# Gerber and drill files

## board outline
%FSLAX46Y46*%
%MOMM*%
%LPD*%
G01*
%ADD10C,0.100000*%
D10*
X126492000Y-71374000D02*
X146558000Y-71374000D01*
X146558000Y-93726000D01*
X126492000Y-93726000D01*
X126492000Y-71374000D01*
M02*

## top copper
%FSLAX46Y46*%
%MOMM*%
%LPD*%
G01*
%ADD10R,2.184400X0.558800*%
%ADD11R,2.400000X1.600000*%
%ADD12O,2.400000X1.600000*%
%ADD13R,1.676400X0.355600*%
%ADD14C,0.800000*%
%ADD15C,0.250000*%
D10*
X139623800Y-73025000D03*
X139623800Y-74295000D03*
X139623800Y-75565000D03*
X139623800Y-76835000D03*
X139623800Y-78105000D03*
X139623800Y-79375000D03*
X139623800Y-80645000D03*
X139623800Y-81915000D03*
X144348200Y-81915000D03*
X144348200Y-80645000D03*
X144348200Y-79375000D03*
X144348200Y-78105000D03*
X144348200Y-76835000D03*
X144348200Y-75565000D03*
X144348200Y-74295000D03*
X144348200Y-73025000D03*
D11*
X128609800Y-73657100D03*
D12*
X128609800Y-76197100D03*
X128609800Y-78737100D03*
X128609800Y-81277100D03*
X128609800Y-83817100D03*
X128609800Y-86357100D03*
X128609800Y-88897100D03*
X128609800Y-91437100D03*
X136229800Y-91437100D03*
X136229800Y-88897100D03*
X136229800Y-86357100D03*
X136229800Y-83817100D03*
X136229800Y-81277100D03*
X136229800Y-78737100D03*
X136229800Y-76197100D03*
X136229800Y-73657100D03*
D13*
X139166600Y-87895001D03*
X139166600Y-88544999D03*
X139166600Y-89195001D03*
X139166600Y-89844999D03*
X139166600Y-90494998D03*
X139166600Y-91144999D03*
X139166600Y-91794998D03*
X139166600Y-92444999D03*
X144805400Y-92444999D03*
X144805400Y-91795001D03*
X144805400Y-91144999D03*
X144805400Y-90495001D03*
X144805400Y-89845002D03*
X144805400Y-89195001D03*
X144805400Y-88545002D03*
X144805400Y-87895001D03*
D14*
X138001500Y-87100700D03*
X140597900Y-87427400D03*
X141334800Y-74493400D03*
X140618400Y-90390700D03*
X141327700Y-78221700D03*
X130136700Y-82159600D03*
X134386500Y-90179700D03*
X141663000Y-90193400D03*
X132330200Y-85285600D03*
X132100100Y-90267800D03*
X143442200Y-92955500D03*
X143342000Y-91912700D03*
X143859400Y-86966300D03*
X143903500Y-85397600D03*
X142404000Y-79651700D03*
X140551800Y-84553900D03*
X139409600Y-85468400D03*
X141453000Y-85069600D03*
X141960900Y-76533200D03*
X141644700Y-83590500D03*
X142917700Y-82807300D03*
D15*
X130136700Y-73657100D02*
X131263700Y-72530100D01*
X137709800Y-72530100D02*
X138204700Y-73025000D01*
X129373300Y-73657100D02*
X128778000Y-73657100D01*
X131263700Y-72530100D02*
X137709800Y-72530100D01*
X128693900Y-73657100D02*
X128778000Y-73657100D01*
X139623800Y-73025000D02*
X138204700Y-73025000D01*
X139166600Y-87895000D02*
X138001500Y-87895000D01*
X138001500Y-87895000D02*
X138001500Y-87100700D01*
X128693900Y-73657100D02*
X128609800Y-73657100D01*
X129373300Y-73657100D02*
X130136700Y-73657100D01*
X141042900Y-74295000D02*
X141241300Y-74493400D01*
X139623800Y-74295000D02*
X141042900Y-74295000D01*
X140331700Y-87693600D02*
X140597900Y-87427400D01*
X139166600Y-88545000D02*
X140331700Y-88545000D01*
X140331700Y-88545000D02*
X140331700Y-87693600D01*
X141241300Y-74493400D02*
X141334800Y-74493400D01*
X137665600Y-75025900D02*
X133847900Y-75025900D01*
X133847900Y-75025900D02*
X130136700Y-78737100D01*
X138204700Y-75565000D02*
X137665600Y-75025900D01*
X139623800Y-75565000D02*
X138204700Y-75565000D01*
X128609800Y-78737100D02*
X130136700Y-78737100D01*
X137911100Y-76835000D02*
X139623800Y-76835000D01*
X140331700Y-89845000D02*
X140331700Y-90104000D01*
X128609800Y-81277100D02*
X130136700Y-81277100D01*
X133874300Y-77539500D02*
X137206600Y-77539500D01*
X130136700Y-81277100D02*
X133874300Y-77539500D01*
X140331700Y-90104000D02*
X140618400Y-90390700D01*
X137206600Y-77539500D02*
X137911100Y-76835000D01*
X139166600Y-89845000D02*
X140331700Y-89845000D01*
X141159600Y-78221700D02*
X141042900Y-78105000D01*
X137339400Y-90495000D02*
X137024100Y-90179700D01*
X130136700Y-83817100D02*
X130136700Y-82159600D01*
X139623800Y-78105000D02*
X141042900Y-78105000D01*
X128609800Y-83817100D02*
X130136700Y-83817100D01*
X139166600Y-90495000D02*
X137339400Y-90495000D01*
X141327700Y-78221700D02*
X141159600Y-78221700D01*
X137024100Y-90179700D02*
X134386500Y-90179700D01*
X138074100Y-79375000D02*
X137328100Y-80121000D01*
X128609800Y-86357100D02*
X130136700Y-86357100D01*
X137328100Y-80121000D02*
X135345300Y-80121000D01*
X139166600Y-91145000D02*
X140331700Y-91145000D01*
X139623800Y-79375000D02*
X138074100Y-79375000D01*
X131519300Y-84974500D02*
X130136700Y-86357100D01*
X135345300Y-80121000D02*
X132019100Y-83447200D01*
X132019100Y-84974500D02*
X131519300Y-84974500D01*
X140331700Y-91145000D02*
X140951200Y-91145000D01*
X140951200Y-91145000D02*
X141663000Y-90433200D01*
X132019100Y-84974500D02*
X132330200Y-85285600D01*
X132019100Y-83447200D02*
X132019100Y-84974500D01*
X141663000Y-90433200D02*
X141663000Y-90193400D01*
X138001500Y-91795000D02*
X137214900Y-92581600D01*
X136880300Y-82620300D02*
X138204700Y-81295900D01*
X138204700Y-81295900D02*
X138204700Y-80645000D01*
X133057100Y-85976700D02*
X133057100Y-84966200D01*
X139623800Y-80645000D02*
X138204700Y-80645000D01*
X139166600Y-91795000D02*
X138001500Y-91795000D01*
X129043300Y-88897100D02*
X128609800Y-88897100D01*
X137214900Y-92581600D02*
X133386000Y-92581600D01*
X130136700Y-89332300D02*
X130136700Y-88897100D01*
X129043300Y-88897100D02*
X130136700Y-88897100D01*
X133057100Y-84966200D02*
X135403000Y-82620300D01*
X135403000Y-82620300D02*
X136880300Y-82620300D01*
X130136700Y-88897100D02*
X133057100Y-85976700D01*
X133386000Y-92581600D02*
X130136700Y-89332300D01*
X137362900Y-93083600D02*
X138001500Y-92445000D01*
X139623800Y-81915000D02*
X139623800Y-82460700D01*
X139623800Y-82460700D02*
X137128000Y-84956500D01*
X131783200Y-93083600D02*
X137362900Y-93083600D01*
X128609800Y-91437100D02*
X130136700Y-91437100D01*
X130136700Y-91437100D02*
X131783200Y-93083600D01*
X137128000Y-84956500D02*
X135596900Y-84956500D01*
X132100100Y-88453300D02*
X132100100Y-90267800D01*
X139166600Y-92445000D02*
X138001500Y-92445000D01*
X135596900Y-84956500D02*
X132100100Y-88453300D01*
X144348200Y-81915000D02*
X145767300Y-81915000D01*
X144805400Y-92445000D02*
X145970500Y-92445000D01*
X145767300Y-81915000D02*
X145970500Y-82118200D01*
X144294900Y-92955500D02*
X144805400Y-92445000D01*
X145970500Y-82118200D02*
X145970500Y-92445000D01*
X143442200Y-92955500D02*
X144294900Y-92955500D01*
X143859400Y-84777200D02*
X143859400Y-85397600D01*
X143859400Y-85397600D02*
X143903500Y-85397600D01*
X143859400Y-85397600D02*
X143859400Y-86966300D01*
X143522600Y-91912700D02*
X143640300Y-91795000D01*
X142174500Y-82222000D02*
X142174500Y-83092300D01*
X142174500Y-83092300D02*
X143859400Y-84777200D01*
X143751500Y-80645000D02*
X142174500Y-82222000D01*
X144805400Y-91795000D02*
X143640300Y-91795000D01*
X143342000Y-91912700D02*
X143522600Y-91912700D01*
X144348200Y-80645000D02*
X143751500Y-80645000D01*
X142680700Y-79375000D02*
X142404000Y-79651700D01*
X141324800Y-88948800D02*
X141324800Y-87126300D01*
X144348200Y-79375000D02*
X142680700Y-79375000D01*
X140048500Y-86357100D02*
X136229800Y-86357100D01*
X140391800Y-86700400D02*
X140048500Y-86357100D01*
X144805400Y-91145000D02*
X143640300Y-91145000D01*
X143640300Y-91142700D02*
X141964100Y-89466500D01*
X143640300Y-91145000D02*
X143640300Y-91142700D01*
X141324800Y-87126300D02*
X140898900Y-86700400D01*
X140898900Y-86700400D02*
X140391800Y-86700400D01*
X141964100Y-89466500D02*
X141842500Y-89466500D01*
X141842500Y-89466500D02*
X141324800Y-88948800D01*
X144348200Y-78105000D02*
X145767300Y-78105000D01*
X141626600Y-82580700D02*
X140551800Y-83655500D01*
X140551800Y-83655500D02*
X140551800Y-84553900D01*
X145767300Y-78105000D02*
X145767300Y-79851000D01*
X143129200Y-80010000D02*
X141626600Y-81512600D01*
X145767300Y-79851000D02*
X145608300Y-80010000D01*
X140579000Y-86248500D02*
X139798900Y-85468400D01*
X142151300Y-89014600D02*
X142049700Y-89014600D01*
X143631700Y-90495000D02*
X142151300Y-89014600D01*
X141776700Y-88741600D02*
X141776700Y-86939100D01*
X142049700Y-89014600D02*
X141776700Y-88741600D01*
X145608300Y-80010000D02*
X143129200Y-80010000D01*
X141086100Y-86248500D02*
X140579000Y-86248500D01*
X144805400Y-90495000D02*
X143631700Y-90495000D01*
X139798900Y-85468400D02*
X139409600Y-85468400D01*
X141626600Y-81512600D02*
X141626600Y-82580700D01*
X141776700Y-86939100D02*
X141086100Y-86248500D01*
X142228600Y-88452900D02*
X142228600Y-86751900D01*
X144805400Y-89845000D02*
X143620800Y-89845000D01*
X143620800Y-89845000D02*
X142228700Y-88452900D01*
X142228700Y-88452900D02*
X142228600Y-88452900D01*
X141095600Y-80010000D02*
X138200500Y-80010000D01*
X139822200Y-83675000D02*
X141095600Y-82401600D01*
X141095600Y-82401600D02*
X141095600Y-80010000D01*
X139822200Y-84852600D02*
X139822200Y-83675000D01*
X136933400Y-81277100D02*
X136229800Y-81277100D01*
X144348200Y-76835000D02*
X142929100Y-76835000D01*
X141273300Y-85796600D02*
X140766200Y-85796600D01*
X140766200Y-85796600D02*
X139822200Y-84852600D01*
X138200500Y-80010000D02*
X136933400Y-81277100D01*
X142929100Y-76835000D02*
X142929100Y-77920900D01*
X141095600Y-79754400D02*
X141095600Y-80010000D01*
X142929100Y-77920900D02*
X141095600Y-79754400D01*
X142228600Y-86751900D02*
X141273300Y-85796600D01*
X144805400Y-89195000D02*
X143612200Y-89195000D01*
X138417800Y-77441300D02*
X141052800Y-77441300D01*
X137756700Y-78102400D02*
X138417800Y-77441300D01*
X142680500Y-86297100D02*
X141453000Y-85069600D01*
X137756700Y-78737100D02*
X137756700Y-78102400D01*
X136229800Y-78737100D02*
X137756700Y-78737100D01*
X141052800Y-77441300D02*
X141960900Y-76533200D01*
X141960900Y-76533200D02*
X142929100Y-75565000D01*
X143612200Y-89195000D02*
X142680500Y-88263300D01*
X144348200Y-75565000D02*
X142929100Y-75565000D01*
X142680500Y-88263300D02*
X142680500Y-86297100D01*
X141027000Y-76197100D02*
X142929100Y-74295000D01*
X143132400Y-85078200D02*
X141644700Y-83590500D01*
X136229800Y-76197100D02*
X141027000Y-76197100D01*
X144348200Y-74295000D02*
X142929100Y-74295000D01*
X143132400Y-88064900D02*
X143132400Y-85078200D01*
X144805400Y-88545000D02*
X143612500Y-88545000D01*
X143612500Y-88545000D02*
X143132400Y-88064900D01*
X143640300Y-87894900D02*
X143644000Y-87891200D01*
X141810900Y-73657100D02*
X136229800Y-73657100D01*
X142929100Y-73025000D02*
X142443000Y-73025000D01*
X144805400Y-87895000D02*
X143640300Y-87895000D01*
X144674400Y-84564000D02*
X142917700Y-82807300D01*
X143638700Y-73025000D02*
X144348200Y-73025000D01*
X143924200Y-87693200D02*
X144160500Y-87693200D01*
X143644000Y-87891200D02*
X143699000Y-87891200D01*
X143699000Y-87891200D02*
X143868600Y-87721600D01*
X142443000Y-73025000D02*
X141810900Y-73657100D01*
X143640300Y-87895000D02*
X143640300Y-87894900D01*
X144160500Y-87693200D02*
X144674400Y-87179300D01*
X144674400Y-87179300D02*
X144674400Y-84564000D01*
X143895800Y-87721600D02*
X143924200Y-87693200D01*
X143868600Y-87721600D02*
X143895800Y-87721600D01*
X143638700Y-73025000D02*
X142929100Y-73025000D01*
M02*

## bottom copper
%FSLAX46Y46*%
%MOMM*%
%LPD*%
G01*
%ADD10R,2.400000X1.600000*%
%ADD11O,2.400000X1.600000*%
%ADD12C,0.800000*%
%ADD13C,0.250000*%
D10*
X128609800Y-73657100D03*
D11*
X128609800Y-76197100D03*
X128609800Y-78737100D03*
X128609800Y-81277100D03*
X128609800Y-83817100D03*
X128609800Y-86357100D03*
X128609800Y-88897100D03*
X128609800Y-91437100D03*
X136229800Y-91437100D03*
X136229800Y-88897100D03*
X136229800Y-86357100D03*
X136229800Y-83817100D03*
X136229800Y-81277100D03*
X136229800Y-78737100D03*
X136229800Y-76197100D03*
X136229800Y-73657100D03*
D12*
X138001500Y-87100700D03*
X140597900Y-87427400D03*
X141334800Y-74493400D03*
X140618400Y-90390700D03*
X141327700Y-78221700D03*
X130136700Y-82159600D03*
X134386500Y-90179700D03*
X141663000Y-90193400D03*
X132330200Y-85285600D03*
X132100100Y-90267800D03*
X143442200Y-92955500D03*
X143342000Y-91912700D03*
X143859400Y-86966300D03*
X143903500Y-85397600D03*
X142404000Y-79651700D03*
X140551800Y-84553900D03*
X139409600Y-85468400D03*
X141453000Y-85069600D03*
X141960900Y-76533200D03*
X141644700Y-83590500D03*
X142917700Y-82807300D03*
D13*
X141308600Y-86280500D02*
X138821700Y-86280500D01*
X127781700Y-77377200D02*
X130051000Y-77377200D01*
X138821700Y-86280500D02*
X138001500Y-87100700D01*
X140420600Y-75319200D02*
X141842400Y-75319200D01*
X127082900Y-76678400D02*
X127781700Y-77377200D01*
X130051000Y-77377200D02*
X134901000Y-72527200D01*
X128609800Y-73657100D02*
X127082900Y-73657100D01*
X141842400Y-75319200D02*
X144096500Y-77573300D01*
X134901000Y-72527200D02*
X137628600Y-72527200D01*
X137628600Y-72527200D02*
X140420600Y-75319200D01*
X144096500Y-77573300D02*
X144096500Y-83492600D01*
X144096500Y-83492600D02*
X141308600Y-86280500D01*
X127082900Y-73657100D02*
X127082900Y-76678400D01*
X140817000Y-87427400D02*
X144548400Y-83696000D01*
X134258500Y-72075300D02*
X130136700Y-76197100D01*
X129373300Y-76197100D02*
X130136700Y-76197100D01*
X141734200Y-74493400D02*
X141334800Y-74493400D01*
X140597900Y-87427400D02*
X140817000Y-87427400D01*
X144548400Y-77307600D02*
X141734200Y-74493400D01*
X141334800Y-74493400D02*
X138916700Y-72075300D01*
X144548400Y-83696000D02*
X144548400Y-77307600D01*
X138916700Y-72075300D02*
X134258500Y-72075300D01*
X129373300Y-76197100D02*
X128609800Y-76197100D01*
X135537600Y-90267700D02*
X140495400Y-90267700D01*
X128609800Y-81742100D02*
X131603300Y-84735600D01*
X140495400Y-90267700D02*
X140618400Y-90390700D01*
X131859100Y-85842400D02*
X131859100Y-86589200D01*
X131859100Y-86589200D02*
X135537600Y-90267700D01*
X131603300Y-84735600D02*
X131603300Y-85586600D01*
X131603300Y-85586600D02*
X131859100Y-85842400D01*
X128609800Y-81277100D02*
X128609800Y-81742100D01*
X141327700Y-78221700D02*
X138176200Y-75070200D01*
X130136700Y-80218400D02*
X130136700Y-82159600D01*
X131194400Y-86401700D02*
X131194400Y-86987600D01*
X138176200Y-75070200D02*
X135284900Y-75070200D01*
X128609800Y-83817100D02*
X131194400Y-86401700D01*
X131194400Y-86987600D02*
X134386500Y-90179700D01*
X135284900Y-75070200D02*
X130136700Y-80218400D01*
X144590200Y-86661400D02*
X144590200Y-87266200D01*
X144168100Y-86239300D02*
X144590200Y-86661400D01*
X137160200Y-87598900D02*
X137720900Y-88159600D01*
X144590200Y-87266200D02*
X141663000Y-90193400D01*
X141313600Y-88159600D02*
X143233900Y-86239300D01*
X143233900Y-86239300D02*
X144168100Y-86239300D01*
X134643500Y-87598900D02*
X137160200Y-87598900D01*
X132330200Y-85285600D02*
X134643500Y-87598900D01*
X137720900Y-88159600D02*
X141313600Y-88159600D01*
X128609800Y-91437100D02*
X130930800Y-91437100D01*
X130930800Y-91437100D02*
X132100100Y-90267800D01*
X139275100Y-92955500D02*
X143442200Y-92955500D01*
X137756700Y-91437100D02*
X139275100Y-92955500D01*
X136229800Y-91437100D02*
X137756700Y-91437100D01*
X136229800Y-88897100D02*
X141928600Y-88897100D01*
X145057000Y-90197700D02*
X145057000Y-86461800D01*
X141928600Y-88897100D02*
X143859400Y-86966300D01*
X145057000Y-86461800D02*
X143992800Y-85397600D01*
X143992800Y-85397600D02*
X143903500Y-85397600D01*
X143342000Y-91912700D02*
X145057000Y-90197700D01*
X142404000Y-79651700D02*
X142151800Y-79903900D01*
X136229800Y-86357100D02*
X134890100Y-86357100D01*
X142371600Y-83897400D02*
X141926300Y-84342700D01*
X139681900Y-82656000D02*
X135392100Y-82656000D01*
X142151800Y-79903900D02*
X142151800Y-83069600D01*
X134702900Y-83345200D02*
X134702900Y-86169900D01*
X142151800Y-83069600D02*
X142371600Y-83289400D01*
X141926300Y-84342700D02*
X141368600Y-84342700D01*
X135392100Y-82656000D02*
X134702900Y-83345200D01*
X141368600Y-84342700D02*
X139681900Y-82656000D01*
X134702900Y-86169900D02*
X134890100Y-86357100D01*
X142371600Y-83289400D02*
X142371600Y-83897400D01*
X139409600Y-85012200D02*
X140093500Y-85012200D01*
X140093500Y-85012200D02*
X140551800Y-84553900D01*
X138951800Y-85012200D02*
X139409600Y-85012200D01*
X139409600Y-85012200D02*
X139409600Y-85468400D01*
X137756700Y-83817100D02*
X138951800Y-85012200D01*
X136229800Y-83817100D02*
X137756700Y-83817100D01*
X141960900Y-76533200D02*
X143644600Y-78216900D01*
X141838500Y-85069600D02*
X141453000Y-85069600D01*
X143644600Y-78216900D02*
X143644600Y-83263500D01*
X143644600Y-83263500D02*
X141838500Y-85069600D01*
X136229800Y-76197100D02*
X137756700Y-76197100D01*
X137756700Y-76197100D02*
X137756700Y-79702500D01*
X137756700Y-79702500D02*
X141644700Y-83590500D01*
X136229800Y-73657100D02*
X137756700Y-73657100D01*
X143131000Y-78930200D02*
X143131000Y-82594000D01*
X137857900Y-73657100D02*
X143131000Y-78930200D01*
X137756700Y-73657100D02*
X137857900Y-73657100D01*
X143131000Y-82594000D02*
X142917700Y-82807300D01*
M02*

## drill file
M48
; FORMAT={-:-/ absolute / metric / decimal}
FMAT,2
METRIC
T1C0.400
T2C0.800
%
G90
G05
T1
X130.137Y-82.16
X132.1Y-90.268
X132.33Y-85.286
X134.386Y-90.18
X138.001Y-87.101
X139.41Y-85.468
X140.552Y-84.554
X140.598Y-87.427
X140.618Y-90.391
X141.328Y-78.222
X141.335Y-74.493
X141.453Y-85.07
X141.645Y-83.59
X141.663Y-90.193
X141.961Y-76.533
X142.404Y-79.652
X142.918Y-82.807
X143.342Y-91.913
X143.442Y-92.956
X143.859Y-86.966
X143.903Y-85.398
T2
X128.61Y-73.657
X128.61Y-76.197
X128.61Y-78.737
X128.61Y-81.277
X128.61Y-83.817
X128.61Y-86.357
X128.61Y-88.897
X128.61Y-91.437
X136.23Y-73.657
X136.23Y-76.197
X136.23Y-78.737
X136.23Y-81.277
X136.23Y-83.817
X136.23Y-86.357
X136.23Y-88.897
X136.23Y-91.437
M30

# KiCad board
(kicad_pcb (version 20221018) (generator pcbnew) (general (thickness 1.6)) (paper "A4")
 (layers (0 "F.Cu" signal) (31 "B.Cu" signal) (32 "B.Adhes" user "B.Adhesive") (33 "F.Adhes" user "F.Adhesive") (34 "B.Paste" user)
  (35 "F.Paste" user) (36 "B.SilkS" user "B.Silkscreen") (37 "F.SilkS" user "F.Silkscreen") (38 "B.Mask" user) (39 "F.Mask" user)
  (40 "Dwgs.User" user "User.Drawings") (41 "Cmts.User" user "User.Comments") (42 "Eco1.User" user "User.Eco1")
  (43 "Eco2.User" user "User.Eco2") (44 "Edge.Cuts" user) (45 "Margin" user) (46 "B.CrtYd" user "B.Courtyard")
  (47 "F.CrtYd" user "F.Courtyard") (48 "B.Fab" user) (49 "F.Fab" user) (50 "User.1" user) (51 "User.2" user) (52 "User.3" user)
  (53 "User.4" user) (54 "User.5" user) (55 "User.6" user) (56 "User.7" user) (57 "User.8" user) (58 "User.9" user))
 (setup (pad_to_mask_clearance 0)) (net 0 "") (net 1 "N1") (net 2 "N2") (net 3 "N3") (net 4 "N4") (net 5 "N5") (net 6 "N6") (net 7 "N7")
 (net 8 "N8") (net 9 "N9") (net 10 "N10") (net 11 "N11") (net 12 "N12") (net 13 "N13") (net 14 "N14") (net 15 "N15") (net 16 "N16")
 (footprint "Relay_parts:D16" (layer "F.Cu") (at 141.986 77.47)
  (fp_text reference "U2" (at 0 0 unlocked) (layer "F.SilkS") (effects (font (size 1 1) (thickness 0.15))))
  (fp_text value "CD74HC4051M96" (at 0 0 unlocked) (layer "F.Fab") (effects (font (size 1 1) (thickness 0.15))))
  (pad "1" smd rect (at -2.3622 -4.445) (size 2.1844 0.5588) (layers "F.Cu" "F.Paste" "F.Mask") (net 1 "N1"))
  (pad "2" smd rect (at -2.3622 -3.175) (size 2.1844 0.5588) (layers "F.Cu" "F.Paste" "F.Mask") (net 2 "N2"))
  (pad "3" smd rect (at -2.3622 -1.905) (size 2.1844 0.5588) (layers "F.Cu" "F.Paste" "F.Mask") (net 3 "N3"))
  (pad "4" smd rect (at -2.3622 -0.635) (size 2.1844 0.5588) (layers "F.Cu" "F.Paste" "F.Mask") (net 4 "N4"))
  (pad "5" smd rect (at -2.3622 0.635) (size 2.1844 0.5588) (layers "F.Cu" "F.Paste" "F.Mask") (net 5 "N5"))
  (pad "6" smd rect (at -2.3622 1.905) (size 2.1844 0.5588) (layers "F.Cu" "F.Paste" "F.Mask") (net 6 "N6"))
  (pad "7" smd rect (at -2.3622 3.175) (size 2.1844 0.5588) (layers "F.Cu" "F.Paste" "F.Mask") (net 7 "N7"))
  (pad "8" smd rect (at -2.3622 4.445) (size 2.1844 0.5588) (layers "F.Cu" "F.Paste" "F.Mask") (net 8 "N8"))
  (pad "9" smd rect (at 2.3622 4.445) (size 2.1844 0.5588) (layers "F.Cu" "F.Paste" "F.Mask") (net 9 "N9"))
  (pad "10" smd rect (at 2.3622 3.175) (size 2.1844 0.5588) (layers "F.Cu" "F.Paste" "F.Mask") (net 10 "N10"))
  (pad "11" smd rect (at 2.3622 1.905) (size 2.1844 0.5588) (layers "F.Cu" "F.Paste" "F.Mask") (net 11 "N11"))
  (pad "12" smd rect (at 2.3622 0.635) (size 2.1844 0.5588) (layers "F.Cu" "F.Paste" "F.Mask") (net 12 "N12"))
  (pad "13" smd rect (at 2.3622 -0.635) (size 2.1844 0.5588) (layers "F.Cu" "F.Paste" "F.Mask") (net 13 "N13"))
  (pad "14" smd rect (at 2.3622 -1.905) (size 2.1844 0.5588) (layers "F.Cu" "F.Paste" "F.Mask") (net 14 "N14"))
  (pad "15" smd rect (at 2.3622 -3.175) (size 2.1844 0.5588) (layers "F.Cu" "F.Paste" "F.Mask") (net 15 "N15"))
  (pad "16" smd rect (at 2.3622 -4.445) (size 2.1844 0.5588) (layers "F.Cu" "F.Paste" "F.Mask") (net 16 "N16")))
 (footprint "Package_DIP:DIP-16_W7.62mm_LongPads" (layer "F.Cu") (at 128.6098 73.6571)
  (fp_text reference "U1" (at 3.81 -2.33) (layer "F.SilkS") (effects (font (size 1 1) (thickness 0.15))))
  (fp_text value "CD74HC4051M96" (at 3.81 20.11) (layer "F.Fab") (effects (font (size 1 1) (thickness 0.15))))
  (pad "1" thru_hole rect (at 0 0) (size 2.4 1.6) (drill 0.8) (layers "*.Cu" "*.Mask") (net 1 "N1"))
  (pad "2" thru_hole oval (at 0 2.54) (size 2.4 1.6) (drill 0.8) (layers "*.Cu" "*.Mask") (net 2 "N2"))
  (pad "3" thru_hole oval (at 0 5.08) (size 2.4 1.6) (drill 0.8) (layers "*.Cu" "*.Mask") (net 3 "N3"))
  (pad "4" thru_hole oval (at 0 7.62) (size 2.4 1.6) (drill 0.8) (layers "*.Cu" "*.Mask") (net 4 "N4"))
  (pad "5" thru_hole oval (at 0 10.16) (size 2.4 1.6) (drill 0.8) (layers "*.Cu" "*.Mask") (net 5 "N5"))
  (pad "6" thru_hole oval (at 0 12.7) (size 2.4 1.6) (drill 0.8) (layers "*.Cu" "*.Mask") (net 6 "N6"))
  (pad "7" thru_hole oval (at 0 15.24) (size 2.4 1.6) (drill 0.8) (layers "*.Cu" "*.Mask") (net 7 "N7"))
  (pad "8" thru_hole oval (at 0 17.78) (size 2.4 1.6) (drill 0.8) (layers "*.Cu" "*.Mask") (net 8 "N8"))
  (pad "9" thru_hole oval (at 7.62 17.78) (size 2.4 1.6) (drill 0.8) (layers "*.Cu" "*.Mask") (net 9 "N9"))
  (pad "10" thru_hole oval (at 7.62 15.24) (size 2.4 1.6) (drill 0.8) (layers "*.Cu" "*.Mask") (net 10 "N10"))
  (pad "11" thru_hole oval (at 7.62 12.7) (size 2.4 1.6) (drill 0.8) (layers "*.Cu" "*.Mask") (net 11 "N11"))
  (pad "12" thru_hole oval (at 7.62 10.16) (size 2.4 1.6) (drill 0.8) (layers "*.Cu" "*.Mask") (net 12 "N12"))
  (pad "13" thru_hole oval (at 7.62 7.62) (size 2.4 1.6) (drill 0.8) (layers "*.Cu" "*.Mask") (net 13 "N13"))
  (pad "14" thru_hole oval (at 7.62 5.08) (size 2.4 1.6) (drill 0.8) (layers "*.Cu" "*.Mask") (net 14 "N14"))
  (pad "15" thru_hole oval (at 7.62 2.54) (size 2.4 1.6) (drill 0.8) (layers "*.Cu" "*.Mask") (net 15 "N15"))
  (pad "16" thru_hole oval (at 7.62 0) (size 2.4 1.6) (drill 0.8) (layers "*.Cu" "*.Mask") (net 16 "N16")))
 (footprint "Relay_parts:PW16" (layer "F.Cu") (at 141.986 90.17)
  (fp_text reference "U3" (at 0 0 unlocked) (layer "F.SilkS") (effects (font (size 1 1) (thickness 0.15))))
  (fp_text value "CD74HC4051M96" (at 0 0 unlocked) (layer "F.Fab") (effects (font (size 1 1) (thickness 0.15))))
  (pad "1" smd rect (at -2.8194 -2.274999) (size 1.6764 0.3556) (layers "F.Cu" "F.Paste" "F.Mask") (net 1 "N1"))
  (pad "2" smd rect (at -2.8194 -1.625001) (size 1.6764 0.3556) (layers "F.Cu" "F.Paste" "F.Mask") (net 2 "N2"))
  (pad "3" smd rect (at -2.8194 -0.974999) (size 1.6764 0.3556) (layers "F.Cu" "F.Paste" "F.Mask") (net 3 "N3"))
  (pad "4" smd rect (at -2.8194 -0.325001) (size 1.6764 0.3556) (layers "F.Cu" "F.Paste" "F.Mask") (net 4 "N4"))
  (pad "5" smd rect (at -2.8194 0.324998) (size 1.6764 0.3556) (layers "F.Cu" "F.Paste" "F.Mask") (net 5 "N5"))
  (pad "6" smd rect (at -2.8194 0.974999) (size 1.6764 0.3556) (layers "F.Cu" "F.Paste" "F.Mask") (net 6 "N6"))
  (pad "7" smd rect (at -2.8194 1.624998) (size 1.6764 0.3556) (layers "F.Cu" "F.Paste" "F.Mask") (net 7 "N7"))
  (pad "8" smd rect (at -2.8194 2.274999) (size 1.6764 0.3556) (layers "F.Cu" "F.Paste" "F.Mask") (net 8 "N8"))
  (pad "9" smd rect (at 2.8194 2.274999) (size 1.6764 0.3556) (layers "F.Cu" "F.Paste" "F.Mask") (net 9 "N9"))
  (pad "10" smd rect (at 2.8194 1.625001) (size 1.6764 0.3556) (layers "F.Cu" "F.Paste" "F.Mask") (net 10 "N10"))
  (pad "11" smd rect (at 2.8194 0.974999) (size 1.6764 0.3556) (layers "F.Cu" "F.Paste" "F.Mask") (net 11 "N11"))
  (pad "12" smd rect (at 2.8194 0.325001) (size 1.6764 0.3556) (layers "F.Cu" "F.Paste" "F.Mask") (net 12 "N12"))
  (pad "13" smd rect (at 2.8194 -0.324998) (size 1.6764 0.3556) (layers "F.Cu" "F.Paste" "F.Mask") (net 13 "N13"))
  (pad "14" smd rect (at 2.8194 -0.974999) (size 1.6764 0.3556) (layers "F.Cu" "F.Paste" "F.Mask") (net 14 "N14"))
  (pad "15" smd rect (at 2.8194 -1.624998) (size 1.6764 0.3556) (layers "F.Cu" "F.Paste" "F.Mask") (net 15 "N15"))
  (pad "16" smd rect (at 2.8194 -2.274999) (size 1.6764 0.3556) (layers "F.Cu" "F.Paste" "F.Mask") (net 16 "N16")))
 (gr_rect (start 126.492 71.374) (end 146.558 93.726) (stroke (width 0.1) (type default)) (fill none) (layer "Edge.Cuts"))
 (segment (start 130.1367 73.6571) (end 131.2637 72.5301) (width 0.25) (layer "F.Cu") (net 1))
 (segment (start 137.7098 72.5301) (end 138.2047 73.025) (width 0.25) (layer "F.Cu") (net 1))
 (segment (start 129.3733 73.6571) (end 128.778 73.6571) (width 0.25) (layer "F.Cu") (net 1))
 (segment (start 131.2637 72.5301) (end 137.7098 72.5301) (width 0.25) (layer "F.Cu") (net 1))
 (segment (start 128.6939 73.6571) (end 128.778 73.6571) (width 0.25) (layer "F.Cu") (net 1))
 (segment (start 139.6238 73.025) (end 138.2047 73.025) (width 0.25) (layer "F.Cu") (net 1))
 (segment (start 139.1666 87.895) (end 138.0015 87.895) (width 0.25) (layer "F.Cu") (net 1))
 (segment (start 138.0015 87.895) (end 138.0015 87.1007) (width 0.25) (layer "F.Cu") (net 1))
 (segment (start 128.6939 73.6571) (end 128.6098 73.6571) (width 0.25) (layer "F.Cu") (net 1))
 (segment (start 129.3733 73.6571) (end 130.1367 73.6571) (width 0.25) (layer "F.Cu") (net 1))
 (via (at 138.0015 87.1007) (size 0.8) (drill 0.4) (layers "F.Cu" "B.Cu") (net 1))
 (segment (start 141.3086 86.2805) (end 138.8217 86.2805) (width 0.25) (layer "B.Cu") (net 1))
 (segment (start 127.7817 77.3772) (end 130.051 77.3772) (width 0.25) (layer "B.Cu") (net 1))
 (segment (start 138.8217 86.2805) (end 138.0015 87.1007) (width 0.25) (layer "B.Cu") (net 1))
 (segment (start 140.4206 75.3192) (end 141.8424 75.3192) (width 0.25) (layer "B.Cu") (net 1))
 (segment (start 127.0829 76.6784) (end 127.7817 77.3772) (width 0.25) (layer "B.Cu") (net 1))
 (segment (start 130.051 77.3772) (end 134.901 72.5272) (width 0.25) (layer "B.Cu") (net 1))
 (segment (start 128.6098 73.6571) (end 127.0829 73.6571) (width 0.25) (layer "B.Cu") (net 1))
 (segment (start 141.8424 75.3192) (end 144.0965 77.5733) (width 0.25) (layer "B.Cu") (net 1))
 (segment (start 134.901 72.5272) (end 137.6286 72.5272) (width 0.25) (layer "B.Cu") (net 1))
 (segment (start 137.6286 72.5272) (end 140.4206 75.3192) (width 0.25) (layer "B.Cu") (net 1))
 (segment (start 144.0965 77.5733) (end 144.0965 83.4926) (width 0.25) (layer "B.Cu") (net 1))
 (segment (start 144.0965 83.4926) (end 141.3086 86.2805) (width 0.25) (layer "B.Cu") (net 1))
 (segment (start 127.0829 73.6571) (end 127.0829 76.6784) (width 0.25) (layer "B.Cu") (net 1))
 (segment (start 141.0429 74.295) (end 141.2413 74.4934) (width 0.25) (layer "F.Cu") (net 2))
 (segment (start 139.6238 74.295) (end 141.0429 74.295) (width 0.25) (layer "F.Cu") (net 2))
 (segment (start 140.3317 87.6936) (end 140.5979 87.4274) (width 0.25) (layer "F.Cu") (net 2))
 (segment (start 139.1666 88.545) (end 140.3317 88.545) (width 0.25) (layer "F.Cu") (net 2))
 (segment (start 140.3317 88.545) (end 140.3317 87.6936) (width 0.25) (layer "F.Cu") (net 2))
 (segment (start 141.2413 74.4934) (end 141.3348 74.4934) (width 0.25) (layer "F.Cu") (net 2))
 (via (at 140.5979 87.4274) (size 0.8) (drill 0.4) (layers "F.Cu" "B.Cu") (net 2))
 (via (at 141.3348 74.4934) (size 0.8) (drill 0.4) (layers "F.Cu" "B.Cu") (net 2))
 (segment (start 140.817 87.4274) (end 144.5484 83.696) (width 0.25) (layer "B.Cu") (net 2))
 (segment (start 134.2585 72.0753) (end 130.1367 76.1971) (width 0.25) (layer "B.Cu") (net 2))
 (segment (start 129.3733 76.1971) (end 130.1367 76.1971) (width 0.25) (layer "B.Cu") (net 2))
 (segment (start 141.7342 74.4934) (end 141.3348 74.4934) (width 0.25) (layer "B.Cu") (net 2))
 (segment (start 140.5979 87.4274) (end 140.817 87.4274) (width 0.25) (layer "B.Cu") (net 2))
 (segment (start 144.5484 77.3076) (end 141.7342 74.4934) (width 0.25) (layer "B.Cu") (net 2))
 (segment (start 141.3348 74.4934) (end 138.9167 72.0753) (width 0.25) (layer "B.Cu") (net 2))
 (segment (start 144.5484 83.696) (end 144.5484 77.3076) (width 0.25) (layer "B.Cu") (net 2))
 (segment (start 138.9167 72.0753) (end 134.2585 72.0753) (width 0.25) (layer "B.Cu") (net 2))
 (segment (start 129.3733 76.1971) (end 128.6098 76.1971) (width 0.25) (layer "B.Cu") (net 2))
 (segment (start 137.6656 75.0259) (end 133.8479 75.0259) (width 0.25) (layer "F.Cu") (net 3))
 (segment (start 133.8479 75.0259) (end 130.1367 78.7371) (width 0.25) (layer "F.Cu") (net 3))
 (segment (start 138.2047 75.565) (end 137.6656 75.0259) (width 0.25) (layer "F.Cu") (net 3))
 (segment (start 139.6238 75.565) (end 138.2047 75.565) (width 0.25) (layer "F.Cu") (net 3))
 (segment (start 128.6098 78.7371) (end 130.1367 78.7371) (width 0.25) (layer "F.Cu") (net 3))
 (segment (start 137.9111 76.835) (end 139.6238 76.835) (width 0.25) (layer "F.Cu") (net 4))
 (segment (start 140.3317 89.845) (end 140.3317 90.104) (width 0.25) (layer "F.Cu") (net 4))
 (segment (start 128.6098 81.2771) (end 130.1367 81.2771) (width 0.25) (layer "F.Cu") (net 4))
 (segment (start 133.8743 77.5395) (end 137.2066 77.5395) (width 0.25) (layer "F.Cu") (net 4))
 (segment (start 130.1367 81.2771) (end 133.8743 77.5395) (width 0.25) (layer "F.Cu") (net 4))
 (segment (start 140.3317 90.104) (end 140.6184 90.3907) (width 0.25) (layer "F.Cu") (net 4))
 (segment (start 137.2066 77.5395) (end 137.9111 76.835) (width 0.25) (layer "F.Cu") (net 4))
 (segment (start 139.1666 89.845) (end 140.3317 89.845) (width 0.25) (layer "F.Cu") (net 4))
 (via (at 140.6184 90.3907) (size 0.8) (drill 0.4) (layers "F.Cu" "B.Cu") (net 4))
 (segment (start 135.5376 90.2677) (end 140.4954 90.2677) (width 0.25) (layer "B.Cu") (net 4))
 (segment (start 128.6098 81.7421) (end 131.6033 84.7356) (width 0.25) (layer "B.Cu") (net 4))
 (segment (start 140.4954 90.2677) (end 140.6184 90.3907) (width 0.25) (layer "B.Cu") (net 4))
 (segment (start 131.8591 85.8424) (end 131.8591 86.5892) (width 0.25) (layer "B.Cu") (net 4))
 (segment (start 131.8591 86.5892) (end 135.5376 90.2677) (width 0.25) (layer "B.Cu") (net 4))
 (segment (start 131.6033 84.7356) (end 131.6033 85.5866) (width 0.25) (layer "B.Cu") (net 4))
 (segment (start 131.6033 85.5866) (end 131.8591 85.8424) (width 0.25) (layer "B.Cu") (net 4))
 (segment (start 128.6098 81.2771) (end 128.6098 81.7421) (width 0.25) (layer "B.Cu") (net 4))
 (segment (start 141.1596 78.2217) (end 141.0429 78.105) (width 0.25) (layer "F.Cu") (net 5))
 (segment (start 137.3394 90.495) (end 137.0241 90.1797) (width 0.25) (layer "F.Cu") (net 5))
 (segment (start 130.1367 83.8171) (end 130.1367 82.1596) (width 0.25) (layer "F.Cu") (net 5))
 (segment (start 139.6238 78.105) (end 141.0429 78.105) (width 0.25) (layer "F.Cu") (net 5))
 (segment (start 128.6098 83.8171) (end 130.1367 83.8171) (width 0.25) (layer "F.Cu") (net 5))
 (segment (start 139.1666 90.495) (end 137.3394 90.495) (width 0.25) (layer "F.Cu") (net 5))
 (segment (start 141.3277 78.2217) (end 141.1596 78.2217) (width 0.25) (layer "F.Cu") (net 5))
 (segment (start 137.0241 90.1797) (end 134.3865 90.1797) (width 0.25) (layer "F.Cu") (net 5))
 (via (at 141.3277 78.2217) (size 0.8) (drill 0.4) (layers "F.Cu" "B.Cu") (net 5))
 (via (at 130.1367 82.1596) (size 0.8) (drill 0.4) (layers "F.Cu" "B.Cu") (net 5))
 (via (at 134.3865 90.1797) (size 0.8) (drill 0.4) (layers "F.Cu" "B.Cu") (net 5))
 (segment (start 141.3277 78.2217) (end 138.1762 75.0702) (width 0.25) (layer "B.Cu") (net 5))
 (segment (start 130.1367 80.2184) (end 130.1367 82.1596) (width 0.25) (layer "B.Cu") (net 5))
 (segment (start 131.1944 86.4017) (end 131.1944 86.9876) (width 0.25) (layer "B.Cu") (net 5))
 (segment (start 138.1762 75.0702) (end 135.2849 75.0702) (width 0.25) (layer "B.Cu") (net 5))
 (segment (start 128.6098 83.8171) (end 131.1944 86.4017) (width 0.25) (layer "B.Cu") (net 5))
 (segment (start 131.1944 86.9876) (end 134.3865 90.1797) (width 0.25) (layer "B.Cu") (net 5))
 (segment (start 135.2849 75.0702) (end 130.1367 80.2184) (width 0.25) (layer "B.Cu") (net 5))
 (segment (start 138.0741 79.375) (end 137.3281 80.121) (width 0.25) (layer "F.Cu") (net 6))
 (segment (start 128.6098 86.3571) (end 130.1367 86.3571) (width 0.25) (layer "F.Cu") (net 6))
 (segment (start 137.3281 80.121) (end 135.3453 80.121) (width 0.25) (layer "F.Cu") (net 6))
 (segment (start 139.1666 91.145) (end 140.3317 91.145) (width 0.25) (layer "F.Cu") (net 6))
 (segment (start 139.6238 79.375) (end 138.0741 79.375) (width 0.25) (layer "F.Cu") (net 6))
 (segment (start 131.5193 84.9745) (end 130.1367 86.3571) (width 0.25) (layer "F.Cu") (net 6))
 (segment (start 135.3453 80.121) (end 132.0191 83.4472) (width 0.25) (layer "F.Cu") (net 6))
 (segment (start 132.0191 84.9745) (end 131.5193 84.9745) (width 0.25) (layer "F.Cu") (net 6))
 (segment (start 140.3317 91.145) (end 140.9512 91.145) (width 0.25) (layer "F.Cu") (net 6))
 (segment (start 140.9512 91.145) (end 141.663 90.4332) (width 0.25) (layer "F.Cu") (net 6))
 (segment (start 132.0191 84.9745) (end 132.3302 85.2856) (width 0.25) (layer "F.Cu") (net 6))
 (segment (start 132.0191 83.4472) (end 132.0191 84.9745) (width 0.25) (layer "F.Cu") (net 6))
 (segment (start 141.663 90.4332) (end 141.663 90.1934) (width 0.25) (layer "F.Cu") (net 6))
 (via (at 141.663 90.1934) (size 0.8) (drill 0.4) (layers "F.Cu" "B.Cu") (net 6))
 (via (at 132.3302 85.2856) (size 0.8) (drill 0.4) (layers "F.Cu" "B.Cu") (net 6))
 (segment (start 144.5902 86.6614) (end 144.5902 87.2662) (width 0.25) (layer "B.Cu") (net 6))
 (segment (start 144.1681 86.2393) (end 144.5902 86.6614) (width 0.25) (layer "B.Cu") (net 6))
 (segment (start 137.1602 87.5989) (end 137.7209 88.1596) (width 0.25) (layer "B.Cu") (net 6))
 (segment (start 144.5902 87.2662) (end 141.663 90.1934) (width 0.25) (layer "B.Cu") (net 6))
 (segment (start 141.3136 88.1596) (end 143.2339 86.2393) (width 0.25) (layer "B.Cu") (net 6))
 (segment (start 143.2339 86.2393) (end 144.1681 86.2393) (width 0.25) (layer "B.Cu") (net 6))
 (segment (start 134.6435 87.5989) (end 137.1602 87.5989) (width 0.25) (layer "B.Cu") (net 6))
 (segment (start 132.3302 85.2856) (end 134.6435 87.5989) (width 0.25) (layer "B.Cu") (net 6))
 (segment (start 137.7209 88.1596) (end 141.3136 88.1596) (width 0.25) (layer "B.Cu") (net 6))
 (segment (start 138.0015 91.795) (end 137.2149 92.5816) (width 0.25) (layer "F.Cu") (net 7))
 (segment (start 136.8803 82.6203) (end 138.2047 81.2959) (width 0.25) (layer "F.Cu") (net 7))
 (segment (start 138.2047 81.2959) (end 138.2047 80.645) (width 0.25) (layer "F.Cu") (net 7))
 (segment (start 133.0571 85.9767) (end 133.0571 84.9662) (width 0.25) (layer "F.Cu") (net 7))
 (segment (start 139.6238 80.645) (end 138.2047 80.645) (width 0.25) (layer "F.Cu") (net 7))
 (segment (start 139.1666 91.795) (end 138.0015 91.795) (width 0.25) (layer "F.Cu") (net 7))
 (segment (start 129.0433 88.8971) (end 128.6098 88.8971) (width 0.25) (layer "F.Cu") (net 7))
 (segment (start 137.2149 92.5816) (end 133.386 92.5816) (width 0.25) (layer "F.Cu") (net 7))
 (segment (start 130.1367 89.3323) (end 130.1367 88.8971) (width 0.25) (layer "F.Cu") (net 7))
 (segment (start 129.0433 88.8971) (end 130.1367 88.8971) (width 0.25) (layer "F.Cu") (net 7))
 (segment (start 133.0571 84.9662) (end 135.403 82.6203) (width 0.25) (layer "F.Cu") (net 7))
 (segment (start 135.403 82.6203) (end 136.8803 82.6203) (width 0.25) (layer "F.Cu") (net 7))
 (segment (start 130.1367 88.8971) (end 133.0571 85.9767) (width 0.25) (layer "F.Cu") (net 7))
 (segment (start 133.386 92.5816) (end 130.1367 89.3323) (width 0.25) (layer "F.Cu") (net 7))
 (segment (start 137.3629 93.0836) (end 138.0015 92.445) (width 0.25) (layer "F.Cu") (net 8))
 (segment (start 139.6238 81.915) (end 139.6238 82.4607) (width 0.25) (layer "F.Cu") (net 8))
 (segment (start 139.6238 82.4607) (end 137.128 84.9565) (width 0.25) (layer "F.Cu") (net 8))
 (segment (start 131.7832 93.0836) (end 137.3629 93.0836) (width 0.25) (layer "F.Cu") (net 8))
 (segment (start 128.6098 91.4371) (end 130.1367 91.4371) (width 0.25) (layer "F.Cu") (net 8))
 (segment (start 130.1367 91.4371) (end 131.7832 93.0836) (width 0.25) (layer "F.Cu") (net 8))
 (segment (start 137.128 84.9565) (end 135.5969 84.9565) (width 0.25) (layer "F.Cu") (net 8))
 (segment (start 132.1001 88.4533) (end 132.1001 90.2678) (width 0.25) (layer "F.Cu") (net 8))
 (segment (start 139.1666 92.445) (end 138.0015 92.445) (width 0.25) (layer "F.Cu") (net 8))
 (segment (start 135.5969 84.9565) (end 132.1001 88.4533) (width 0.25) (layer "F.Cu") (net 8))
 (via (at 132.1001 90.2678) (size 0.8) (drill 0.4) (layers "F.Cu" "B.Cu") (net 8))
 (segment (start 128.6098 91.4371) (end 130.9308 91.4371) (width 0.25) (layer "B.Cu") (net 8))
 (segment (start 130.9308 91.4371) (end 132.1001 90.2678) (width 0.25) (layer "B.Cu") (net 8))
 (segment (start 144.3482 81.915) (end 145.7673 81.915) (width 0.25) (layer "F.Cu") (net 9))
 (segment (start 144.8054 92.445) (end 145.9705 92.445) (width 0.25) (layer "F.Cu") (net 9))
 (segment (start 145.7673 81.915) (end 145.9705 82.1182) (width 0.25) (layer "F.Cu") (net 9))
 (segment (start 144.2949 92.9555) (end 144.8054 92.445) (width 0.25) (layer "F.Cu") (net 9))
 (segment (start 145.9705 82.1182) (end 145.9705 92.445) (width 0.25) (layer "F.Cu") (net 9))
 (segment (start 143.4422 92.9555) (end 144.2949 92.9555) (width 0.25) (layer "F.Cu") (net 9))
 (via (at 143.4422 92.9555) (size 0.8) (drill 0.4) (layers "F.Cu" "B.Cu") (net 9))
 (segment (start 139.2751 92.9555) (end 143.4422 92.9555) (width 0.25) (layer "B.Cu") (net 9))
 (segment (start 137.7567 91.4371) (end 139.2751 92.9555) (width 0.25) (layer "B.Cu") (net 9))
 (segment (start 136.2298 91.4371) (end 137.7567 91.4371) (width 0.25) (layer "B.Cu") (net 9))
 (segment (start 143.8594 84.7772) (end 143.8594 85.3976) (width 0.25) (layer "F.Cu") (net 10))
 (segment (start 143.8594 85.3976) (end 143.9035 85.3976) (width 0.25) (layer "F.Cu") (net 10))
 (segment (start 143.8594 85.3976) (end 143.8594 86.9663) (width 0.25) (layer "F.Cu") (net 10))
 (segment (start 143.5226 91.9127) (end 143.6403 91.795) (width 0.25) (layer "F.Cu") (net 10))
 (segment (start 142.1745 82.222) (end 142.1745 83.0923) (width 0.25) (layer "F.Cu") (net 10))
 (segment (start 142.1745 83.0923) (end 143.8594 84.7772) (width 0.25) (layer "F.Cu") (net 10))
 (segment (start 143.7515 80.645) (end 142.1745 82.222) (width 0.25) (layer "F.Cu") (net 10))
 (segment (start 144.8054 91.795) (end 143.6403 91.795) (width 0.25) (layer "F.Cu") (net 10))
 (segment (start 143.342 91.9127) (end 143.5226 91.9127) (width 0.25) (layer "F.Cu") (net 10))
 (segment (start 144.3482 80.645) (end 143.7515 80.645) (width 0.25) (layer "F.Cu") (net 10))
 (via (at 143.342 91.9127) (size 0.8) (drill 0.4) (layers "F.Cu" "B.Cu") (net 10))
 (via (at 143.8594 86.9663) (size 0.8) (drill 0.4) (layers "F.Cu" "B.Cu") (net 10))
 (via (at 143.9035 85.3976) (size 0.8) (drill 0.4) (layers "F.Cu" "B.Cu") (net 10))
 (segment (start 136.2298 88.8971) (end 141.9286 88.8971) (width 0.25) (layer "B.Cu") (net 10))
 (segment (start 145.057 90.1977) (end 145.057 86.4618) (width 0.25) (layer "B.Cu") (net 10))
 (segment (start 141.9286 88.8971) (end 143.8594 86.9663) (width 0.25) (layer "B.Cu") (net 10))
 (segment (start 145.057 86.4618) (end 143.9928 85.3976) (width 0.25) (layer "B.Cu") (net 10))
 (segment (start 143.9928 85.3976) (end 143.9035 85.3976) (width 0.25) (layer "B.Cu") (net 10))
 (segment (start 143.342 91.9127) (end 145.057 90.1977) (width 0.25) (layer "B.Cu") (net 10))
 (segment (start 142.6807 79.375) (end 142.404 79.6517) (width 0.25) (layer "F.Cu") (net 11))
 (segment (start 141.3248 88.9488) (end 141.3248 87.1263) (width 0.25) (layer "F.Cu") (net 11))
 (segment (start 144.3482 79.375) (end 142.6807 79.375) (width 0.25) (layer "F.Cu") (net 11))
 (segment (start 140.0485 86.3571) (end 136.2298 86.3571) (width 0.25) (layer "F.Cu") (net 11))
 (segment (start 140.3918 86.7004) (end 140.0485 86.3571) (width 0.25) (layer "F.Cu") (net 11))
 (segment (start 144.8054 91.145) (end 143.6403 91.145) (width 0.25) (layer "F.Cu") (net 11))
 (segment (start 143.6403 91.1427) (end 141.9641 89.4665) (width 0.25) (layer "F.Cu") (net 11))
 (segment (start 143.6403 91.145) (end 143.6403 91.1427) (width 0.25) (layer "F.Cu") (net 11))
 (segment (start 141.3248 87.1263) (end 140.8989 86.7004) (width 0.25) (layer "F.Cu") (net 11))
 (segment (start 140.8989 86.7004) (end 140.3918 86.7004) (width 0.25) (layer "F.Cu") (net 11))
 (segment (start 141.9641 89.4665) (end 141.8425 89.4665) (width 0.25) (layer "F.Cu") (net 11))
 (segment (start 141.8425 89.4665) (end 141.3248 88.9488) (width 0.25) (layer "F.Cu") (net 11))
 (via (at 142.404 79.6517) (size 0.8) (drill 0.4) (layers "F.Cu" "B.Cu") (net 11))
 (segment (start 142.404 79.6517) (end 142.1518 79.9039) (width 0.25) (layer "B.Cu") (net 11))
 (segment (start 136.2298 86.3571) (end 134.8901 86.3571) (width 0.25) (layer "B.Cu") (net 11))
 (segment (start 142.3716 83.8974) (end 141.9263 84.3427) (width 0.25) (layer "B.Cu") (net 11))
 (segment (start 139.6819 82.656) (end 135.3921 82.656) (width 0.25) (layer "B.Cu") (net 11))
 (segment (start 142.1518 79.9039) (end 142.1518 83.0696) (width 0.25) (layer "B.Cu") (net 11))
 (segment (start 134.7029 83.3452) (end 134.7029 86.1699) (width 0.25) (layer "B.Cu") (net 11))
 (segment (start 142.1518 83.0696) (end 142.3716 83.2894) (width 0.25) (layer "B.Cu") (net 11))
 (segment (start 141.9263 84.3427) (end 141.3686 84.3427) (width 0.25) (layer "B.Cu") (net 11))
 (segment (start 135.3921 82.656) (end 134.7029 83.3452) (width 0.25) (layer "B.Cu") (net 11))
 (segment (start 141.3686 84.3427) (end 139.6819 82.656) (width 0.25) (layer "B.Cu") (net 11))
 (segment (start 134.7029 86.1699) (end 134.8901 86.3571) (width 0.25) (layer "B.Cu") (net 11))
 (segment (start 142.3716 83.2894) (end 142.3716 83.8974) (width 0.25) (layer "B.Cu") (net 11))
 (segment (start 144.3482 78.105) (end 145.7673 78.105) (width 0.25) (layer "F.Cu") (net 12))
 (segment (start 141.6266 82.5807) (end 140.5518 83.6555) (width 0.25) (layer "F.Cu") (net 12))
 (segment (start 140.5518 83.6555) (end 140.5518 84.5539) (width 0.25) (layer "F.Cu") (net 12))
 (segment (start 145.7673 78.105) (end 145.7673 79.851) (width 0.25) (layer "F.Cu") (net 12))
 (segment (start 143.1292 80.01) (end 141.6266 81.5126) (width 0.25) (layer "F.Cu") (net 12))
 (segment (start 145.7673 79.851) (end 145.6083 80.01) (width 0.25) (layer "F.Cu") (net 12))
 (segment (start 140.579 86.2485) (end 139.7989 85.4684) (width 0.25) (layer "F.Cu") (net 12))
 (segment (start 142.1513 89.0146) (end 142.0497 89.0146) (width 0.25) (layer "F.Cu") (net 12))
 (segment (start 143.6317 90.495) (end 142.1513 89.0146) (width 0.25) (layer "F.Cu") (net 12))
 (segment (start 141.7767 88.7416) (end 141.7767 86.9391) (width 0.25) (layer "F.Cu") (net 12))
 (segment (start 142.0497 89.0146) (end 141.7767 88.7416) (width 0.25) (layer "F.Cu") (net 12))
 (segment (start 145.6083 80.01) (end 143.1292 80.01) (width 0.25) (layer "F.Cu") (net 12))
 (segment (start 141.0861 86.2485) (end 140.579 86.2485) (width 0.25) (layer "F.Cu") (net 12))
 (segment (start 144.8054 90.495) (end 143.6317 90.495) (width 0.25) (layer "F.Cu") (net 12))
 (segment (start 139.7989 85.4684) (end 139.4096 85.4684) (width 0.25) (layer "F.Cu") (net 12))
 (segment (start 141.6266 81.5126) (end 141.6266 82.5807) (width 0.25) (layer "F.Cu") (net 12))
 (segment (start 141.7767 86.9391) (end 141.0861 86.2485) (width 0.25) (layer "F.Cu") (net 12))
 (via (at 140.5518 84.5539) (size 0.8) (drill 0.4) (layers "F.Cu" "B.Cu") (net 12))
 (via (at 139.4096 85.4684) (size 0.8) (drill 0.4) (layers "F.Cu" "B.Cu") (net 12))
 (segment (start 139.4096 85.0122) (end 140.0935 85.0122) (width 0.25) (layer "B.Cu") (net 12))
 (segment (start 140.0935 85.0122) (end 140.5518 84.5539) (width 0.25) (layer "B.Cu") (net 12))
 (segment (start 138.9518 85.0122) (end 139.4096 85.0122) (width 0.25) (layer "B.Cu") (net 12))
 (segment (start 139.4096 85.0122) (end 139.4096 85.4684) (width 0.25) (layer "B.Cu") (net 12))
 (segment (start 137.7567 83.8171) (end 138.9518 85.0122) (width 0.25) (layer "B.Cu") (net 12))
 (segment (start 136.2298 83.8171) (end 137.7567 83.8171) (width 0.25) (layer "B.Cu") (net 12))
 (segment (start 142.2286 88.4529) (end 142.2286 86.7519) (width 0.25) (layer "F.Cu") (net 13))
 (segment (start 144.8054 89.845) (end 143.6208 89.845) (width 0.25) (layer "F.Cu") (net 13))
 (segment (start 143.6208 89.845) (end 142.2287 88.4529) (width 0.25) (layer "F.Cu") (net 13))
 (segment (start 142.2287 88.4529) (end 142.2286 88.4529) (width 0.25) (layer "F.Cu") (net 13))
 (segment (start 141.0956 80.01) (end 138.2005 80.01) (width 0.25) (layer "F.Cu") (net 13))
 (segment (start 139.8222 83.675) (end 141.0956 82.4016) (width 0.25) (layer "F.Cu") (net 13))
 (segment (start 141.0956 82.4016) (end 141.0956 80.01) (width 0.25) (layer "F.Cu") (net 13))
 (segment (start 139.8222 84.8526) (end 139.8222 83.675) (width 0.25) (layer "F.Cu") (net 13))
 (segment (start 136.9334 81.2771) (end 136.2298 81.2771) (width 0.25) (layer "F.Cu") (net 13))
 (segment (start 144.3482 76.835) (end 142.9291 76.835) (width 0.25) (layer "F.Cu") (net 13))
 (segment (start 141.2733 85.7966) (end 140.7662 85.7966) (width 0.25) (layer "F.Cu") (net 13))
 (segment (start 140.7662 85.7966) (end 139.8222 84.8526) (width 0.25) (layer "F.Cu") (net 13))
 (segment (start 138.2005 80.01) (end 136.9334 81.2771) (width 0.25) (layer "F.Cu") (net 13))
 (segment (start 142.9291 76.835) (end 142.9291 77.9209) (width 0.25) (layer "F.Cu") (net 13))
 (segment (start 141.0956 79.7544) (end 141.0956 80.01) (width 0.25) (layer "F.Cu") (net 13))
 (segment (start 142.9291 77.9209) (end 141.0956 79.7544) (width 0.25) (layer "F.Cu") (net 13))
 (segment (start 142.2286 86.7519) (end 141.2733 85.7966) (width 0.25) (layer "F.Cu") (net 13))
 (segment (start 144.8054 89.195) (end 143.6122 89.195) (width 0.25) (layer "F.Cu") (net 14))
 (segment (start 138.4178 77.4413) (end 141.0528 77.4413) (width 0.25) (layer "F.Cu") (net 14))
 (segment (start 137.7567 78.1024) (end 138.4178 77.4413) (width 0.25) (layer "F.Cu") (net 14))
 (segment (start 142.6805 86.2971) (end 141.453 85.0696) (width 0.25) (layer "F.Cu") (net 14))
 (segment (start 137.7567 78.7371) (end 137.7567 78.1024) (width 0.25) (layer "F.Cu") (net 14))
 (segment (start 136.2298 78.7371) (end 137.7567 78.7371) (width 0.25) (layer "F.Cu") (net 14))
 (segment (start 141.0528 77.4413) (end 141.9609 76.5332) (width 0.25) (layer "F.Cu") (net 14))
 (segment (start 141.9609 76.5332) (end 142.9291 75.565) (width 0.25) (layer "F.Cu") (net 14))
 (segment (start 143.6122 89.195) (end 142.6805 88.2633) (width 0.25) (layer "F.Cu") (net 14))
 (segment (start 144.3482 75.565) (end 142.9291 75.565) (width 0.25) (layer "F.Cu") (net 14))
 (segment (start 142.6805 88.2633) (end 142.6805 86.2971) (width 0.25) (layer "F.Cu") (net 14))
 (via (at 141.453 85.0696) (size 0.8) (drill 0.4) (layers "F.Cu" "B.Cu") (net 14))
 (via (at 141.9609 76.5332) (size 0.8) (drill 0.4) (layers "F.Cu" "B.Cu") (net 14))
 (segment (start 141.9609 76.5332) (end 143.6446 78.2169) (width 0.25) (layer "B.Cu") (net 14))
 (segment (start 141.8385 85.0696) (end 141.453 85.0696) (width 0.25) (layer "B.Cu") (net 14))
 (segment (start 143.6446 78.2169) (end 143.6446 83.2635) (width 0.25) (layer "B.Cu") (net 14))
 (segment (start 143.6446 83.2635) (end 141.8385 85.0696) (width 0.25) (layer "B.Cu") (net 14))
 (segment (start 141.027 76.1971) (end 142.9291 74.295) (width 0.25) (layer "F.Cu") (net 15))
 (segment (start 143.1324 85.0782) (end 141.6447 83.5905) (width 0.25) (layer "F.Cu") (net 15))
 (segment (start 136.2298 76.1971) (end 141.027 76.1971) (width 0.25) (layer "F.Cu") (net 15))
 (segment (start 144.3482 74.295) (end 142.9291 74.295) (width 0.25) (layer "F.Cu") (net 15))
 (segment (start 143.1324 88.0649) (end 143.1324 85.0782) (width 0.25) (layer "F.Cu") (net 15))
 (segment (start 144.8054 88.545) (end 143.6125 88.545) (width 0.25) (layer "F.Cu") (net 15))
 (segment (start 143.6125 88.545) (end 143.1324 88.0649) (width 0.25) (layer "F.Cu") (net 15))
 (via (at 141.6447 83.5905) (size 0.8) (drill 0.4) (layers "F.Cu" "B.Cu") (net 15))
 (segment (start 136.2298 76.1971) (end 137.7567 76.1971) (width 0.25) (layer "B.Cu") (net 15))
 (segment (start 137.7567 76.1971) (end 137.7567 79.7025) (width 0.25) (layer "B.Cu") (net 15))
 (segment (start 137.7567 79.7025) (end 141.6447 83.5905) (width 0.25) (layer "B.Cu") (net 15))
 (segment (start 143.6403 87.8949) (end 143.644 87.8912) (width 0.25) (layer "F.Cu") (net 16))
 (segment (start 141.8109 73.6571) (end 136.2298 73.6571) (width 0.25) (layer "F.Cu") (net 16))
 (segment (start 142.9291 73.025) (end 142.443 73.025) (width 0.25) (layer "F.Cu") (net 16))
 (segment (start 144.8054 87.895) (end 143.6403 87.895) (width 0.25) (layer "F.Cu") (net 16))
 (segment (start 144.6744 84.564) (end 142.9177 82.8073) (width 0.25) (layer "F.Cu") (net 16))
 (segment (start 143.6387 73.025) (end 144.3482 73.025) (width 0.25) (layer "F.Cu") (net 16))
 (segment (start 143.9242 87.6932) (end 144.1605 87.6932) (width 0.25) (layer "F.Cu") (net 16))
 (segment (start 143.644 87.8912) (end 143.699 87.8912) (width 0.25) (layer "F.Cu") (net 16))
 (segment (start 143.699 87.8912) (end 143.8686 87.7216) (width 0.25) (layer "F.Cu") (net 16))
 (segment (start 142.443 73.025) (end 141.8109 73.6571) (width 0.25) (layer "F.Cu") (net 16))
 (segment (start 143.6403 87.895) (end 143.6403 87.8949) (width 0.25) (layer "F.Cu") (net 16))
 (segment (start 144.1605 87.6932) (end 144.6744 87.1793) (width 0.25) (layer "F.Cu") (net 16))
 (segment (start 144.6744 87.1793) (end 144.6744 84.564) (width 0.25) (layer "F.Cu") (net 16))
 (segment (start 143.8958 87.7216) (end 143.9242 87.6932) (width 0.25) (layer "F.Cu") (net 16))
 (segment (start 143.8686 87.7216) (end 143.8958 87.7216) (width 0.25) (layer "F.Cu") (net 16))
 (segment (start 143.6387 73.025) (end 142.9291 73.025) (width 0.25) (layer "F.Cu") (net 16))
 (via (at 142.9177 82.8073) (size 0.8) (drill 0.4) (layers "F.Cu" "B.Cu") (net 16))
 (segment (start 136.2298 73.6571) (end 137.7567 73.6571) (width 0.25) (layer "B.Cu") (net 16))
 (segment (start 143.131 78.9302) (end 143.131 82.594) (width 0.25) (layer "B.Cu") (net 16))
 (segment (start 137.8579 73.6571) (end 143.131 78.9302) (width 0.25) (layer "B.Cu") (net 16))
 (segment (start 137.7567 73.6571) (end 137.8579 73.6571) (width 0.25) (layer "B.Cu") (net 16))
 (segment (start 143.131 82.594) (end 142.9177 82.8073) (width 0.25) (layer "B.Cu") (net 16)))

